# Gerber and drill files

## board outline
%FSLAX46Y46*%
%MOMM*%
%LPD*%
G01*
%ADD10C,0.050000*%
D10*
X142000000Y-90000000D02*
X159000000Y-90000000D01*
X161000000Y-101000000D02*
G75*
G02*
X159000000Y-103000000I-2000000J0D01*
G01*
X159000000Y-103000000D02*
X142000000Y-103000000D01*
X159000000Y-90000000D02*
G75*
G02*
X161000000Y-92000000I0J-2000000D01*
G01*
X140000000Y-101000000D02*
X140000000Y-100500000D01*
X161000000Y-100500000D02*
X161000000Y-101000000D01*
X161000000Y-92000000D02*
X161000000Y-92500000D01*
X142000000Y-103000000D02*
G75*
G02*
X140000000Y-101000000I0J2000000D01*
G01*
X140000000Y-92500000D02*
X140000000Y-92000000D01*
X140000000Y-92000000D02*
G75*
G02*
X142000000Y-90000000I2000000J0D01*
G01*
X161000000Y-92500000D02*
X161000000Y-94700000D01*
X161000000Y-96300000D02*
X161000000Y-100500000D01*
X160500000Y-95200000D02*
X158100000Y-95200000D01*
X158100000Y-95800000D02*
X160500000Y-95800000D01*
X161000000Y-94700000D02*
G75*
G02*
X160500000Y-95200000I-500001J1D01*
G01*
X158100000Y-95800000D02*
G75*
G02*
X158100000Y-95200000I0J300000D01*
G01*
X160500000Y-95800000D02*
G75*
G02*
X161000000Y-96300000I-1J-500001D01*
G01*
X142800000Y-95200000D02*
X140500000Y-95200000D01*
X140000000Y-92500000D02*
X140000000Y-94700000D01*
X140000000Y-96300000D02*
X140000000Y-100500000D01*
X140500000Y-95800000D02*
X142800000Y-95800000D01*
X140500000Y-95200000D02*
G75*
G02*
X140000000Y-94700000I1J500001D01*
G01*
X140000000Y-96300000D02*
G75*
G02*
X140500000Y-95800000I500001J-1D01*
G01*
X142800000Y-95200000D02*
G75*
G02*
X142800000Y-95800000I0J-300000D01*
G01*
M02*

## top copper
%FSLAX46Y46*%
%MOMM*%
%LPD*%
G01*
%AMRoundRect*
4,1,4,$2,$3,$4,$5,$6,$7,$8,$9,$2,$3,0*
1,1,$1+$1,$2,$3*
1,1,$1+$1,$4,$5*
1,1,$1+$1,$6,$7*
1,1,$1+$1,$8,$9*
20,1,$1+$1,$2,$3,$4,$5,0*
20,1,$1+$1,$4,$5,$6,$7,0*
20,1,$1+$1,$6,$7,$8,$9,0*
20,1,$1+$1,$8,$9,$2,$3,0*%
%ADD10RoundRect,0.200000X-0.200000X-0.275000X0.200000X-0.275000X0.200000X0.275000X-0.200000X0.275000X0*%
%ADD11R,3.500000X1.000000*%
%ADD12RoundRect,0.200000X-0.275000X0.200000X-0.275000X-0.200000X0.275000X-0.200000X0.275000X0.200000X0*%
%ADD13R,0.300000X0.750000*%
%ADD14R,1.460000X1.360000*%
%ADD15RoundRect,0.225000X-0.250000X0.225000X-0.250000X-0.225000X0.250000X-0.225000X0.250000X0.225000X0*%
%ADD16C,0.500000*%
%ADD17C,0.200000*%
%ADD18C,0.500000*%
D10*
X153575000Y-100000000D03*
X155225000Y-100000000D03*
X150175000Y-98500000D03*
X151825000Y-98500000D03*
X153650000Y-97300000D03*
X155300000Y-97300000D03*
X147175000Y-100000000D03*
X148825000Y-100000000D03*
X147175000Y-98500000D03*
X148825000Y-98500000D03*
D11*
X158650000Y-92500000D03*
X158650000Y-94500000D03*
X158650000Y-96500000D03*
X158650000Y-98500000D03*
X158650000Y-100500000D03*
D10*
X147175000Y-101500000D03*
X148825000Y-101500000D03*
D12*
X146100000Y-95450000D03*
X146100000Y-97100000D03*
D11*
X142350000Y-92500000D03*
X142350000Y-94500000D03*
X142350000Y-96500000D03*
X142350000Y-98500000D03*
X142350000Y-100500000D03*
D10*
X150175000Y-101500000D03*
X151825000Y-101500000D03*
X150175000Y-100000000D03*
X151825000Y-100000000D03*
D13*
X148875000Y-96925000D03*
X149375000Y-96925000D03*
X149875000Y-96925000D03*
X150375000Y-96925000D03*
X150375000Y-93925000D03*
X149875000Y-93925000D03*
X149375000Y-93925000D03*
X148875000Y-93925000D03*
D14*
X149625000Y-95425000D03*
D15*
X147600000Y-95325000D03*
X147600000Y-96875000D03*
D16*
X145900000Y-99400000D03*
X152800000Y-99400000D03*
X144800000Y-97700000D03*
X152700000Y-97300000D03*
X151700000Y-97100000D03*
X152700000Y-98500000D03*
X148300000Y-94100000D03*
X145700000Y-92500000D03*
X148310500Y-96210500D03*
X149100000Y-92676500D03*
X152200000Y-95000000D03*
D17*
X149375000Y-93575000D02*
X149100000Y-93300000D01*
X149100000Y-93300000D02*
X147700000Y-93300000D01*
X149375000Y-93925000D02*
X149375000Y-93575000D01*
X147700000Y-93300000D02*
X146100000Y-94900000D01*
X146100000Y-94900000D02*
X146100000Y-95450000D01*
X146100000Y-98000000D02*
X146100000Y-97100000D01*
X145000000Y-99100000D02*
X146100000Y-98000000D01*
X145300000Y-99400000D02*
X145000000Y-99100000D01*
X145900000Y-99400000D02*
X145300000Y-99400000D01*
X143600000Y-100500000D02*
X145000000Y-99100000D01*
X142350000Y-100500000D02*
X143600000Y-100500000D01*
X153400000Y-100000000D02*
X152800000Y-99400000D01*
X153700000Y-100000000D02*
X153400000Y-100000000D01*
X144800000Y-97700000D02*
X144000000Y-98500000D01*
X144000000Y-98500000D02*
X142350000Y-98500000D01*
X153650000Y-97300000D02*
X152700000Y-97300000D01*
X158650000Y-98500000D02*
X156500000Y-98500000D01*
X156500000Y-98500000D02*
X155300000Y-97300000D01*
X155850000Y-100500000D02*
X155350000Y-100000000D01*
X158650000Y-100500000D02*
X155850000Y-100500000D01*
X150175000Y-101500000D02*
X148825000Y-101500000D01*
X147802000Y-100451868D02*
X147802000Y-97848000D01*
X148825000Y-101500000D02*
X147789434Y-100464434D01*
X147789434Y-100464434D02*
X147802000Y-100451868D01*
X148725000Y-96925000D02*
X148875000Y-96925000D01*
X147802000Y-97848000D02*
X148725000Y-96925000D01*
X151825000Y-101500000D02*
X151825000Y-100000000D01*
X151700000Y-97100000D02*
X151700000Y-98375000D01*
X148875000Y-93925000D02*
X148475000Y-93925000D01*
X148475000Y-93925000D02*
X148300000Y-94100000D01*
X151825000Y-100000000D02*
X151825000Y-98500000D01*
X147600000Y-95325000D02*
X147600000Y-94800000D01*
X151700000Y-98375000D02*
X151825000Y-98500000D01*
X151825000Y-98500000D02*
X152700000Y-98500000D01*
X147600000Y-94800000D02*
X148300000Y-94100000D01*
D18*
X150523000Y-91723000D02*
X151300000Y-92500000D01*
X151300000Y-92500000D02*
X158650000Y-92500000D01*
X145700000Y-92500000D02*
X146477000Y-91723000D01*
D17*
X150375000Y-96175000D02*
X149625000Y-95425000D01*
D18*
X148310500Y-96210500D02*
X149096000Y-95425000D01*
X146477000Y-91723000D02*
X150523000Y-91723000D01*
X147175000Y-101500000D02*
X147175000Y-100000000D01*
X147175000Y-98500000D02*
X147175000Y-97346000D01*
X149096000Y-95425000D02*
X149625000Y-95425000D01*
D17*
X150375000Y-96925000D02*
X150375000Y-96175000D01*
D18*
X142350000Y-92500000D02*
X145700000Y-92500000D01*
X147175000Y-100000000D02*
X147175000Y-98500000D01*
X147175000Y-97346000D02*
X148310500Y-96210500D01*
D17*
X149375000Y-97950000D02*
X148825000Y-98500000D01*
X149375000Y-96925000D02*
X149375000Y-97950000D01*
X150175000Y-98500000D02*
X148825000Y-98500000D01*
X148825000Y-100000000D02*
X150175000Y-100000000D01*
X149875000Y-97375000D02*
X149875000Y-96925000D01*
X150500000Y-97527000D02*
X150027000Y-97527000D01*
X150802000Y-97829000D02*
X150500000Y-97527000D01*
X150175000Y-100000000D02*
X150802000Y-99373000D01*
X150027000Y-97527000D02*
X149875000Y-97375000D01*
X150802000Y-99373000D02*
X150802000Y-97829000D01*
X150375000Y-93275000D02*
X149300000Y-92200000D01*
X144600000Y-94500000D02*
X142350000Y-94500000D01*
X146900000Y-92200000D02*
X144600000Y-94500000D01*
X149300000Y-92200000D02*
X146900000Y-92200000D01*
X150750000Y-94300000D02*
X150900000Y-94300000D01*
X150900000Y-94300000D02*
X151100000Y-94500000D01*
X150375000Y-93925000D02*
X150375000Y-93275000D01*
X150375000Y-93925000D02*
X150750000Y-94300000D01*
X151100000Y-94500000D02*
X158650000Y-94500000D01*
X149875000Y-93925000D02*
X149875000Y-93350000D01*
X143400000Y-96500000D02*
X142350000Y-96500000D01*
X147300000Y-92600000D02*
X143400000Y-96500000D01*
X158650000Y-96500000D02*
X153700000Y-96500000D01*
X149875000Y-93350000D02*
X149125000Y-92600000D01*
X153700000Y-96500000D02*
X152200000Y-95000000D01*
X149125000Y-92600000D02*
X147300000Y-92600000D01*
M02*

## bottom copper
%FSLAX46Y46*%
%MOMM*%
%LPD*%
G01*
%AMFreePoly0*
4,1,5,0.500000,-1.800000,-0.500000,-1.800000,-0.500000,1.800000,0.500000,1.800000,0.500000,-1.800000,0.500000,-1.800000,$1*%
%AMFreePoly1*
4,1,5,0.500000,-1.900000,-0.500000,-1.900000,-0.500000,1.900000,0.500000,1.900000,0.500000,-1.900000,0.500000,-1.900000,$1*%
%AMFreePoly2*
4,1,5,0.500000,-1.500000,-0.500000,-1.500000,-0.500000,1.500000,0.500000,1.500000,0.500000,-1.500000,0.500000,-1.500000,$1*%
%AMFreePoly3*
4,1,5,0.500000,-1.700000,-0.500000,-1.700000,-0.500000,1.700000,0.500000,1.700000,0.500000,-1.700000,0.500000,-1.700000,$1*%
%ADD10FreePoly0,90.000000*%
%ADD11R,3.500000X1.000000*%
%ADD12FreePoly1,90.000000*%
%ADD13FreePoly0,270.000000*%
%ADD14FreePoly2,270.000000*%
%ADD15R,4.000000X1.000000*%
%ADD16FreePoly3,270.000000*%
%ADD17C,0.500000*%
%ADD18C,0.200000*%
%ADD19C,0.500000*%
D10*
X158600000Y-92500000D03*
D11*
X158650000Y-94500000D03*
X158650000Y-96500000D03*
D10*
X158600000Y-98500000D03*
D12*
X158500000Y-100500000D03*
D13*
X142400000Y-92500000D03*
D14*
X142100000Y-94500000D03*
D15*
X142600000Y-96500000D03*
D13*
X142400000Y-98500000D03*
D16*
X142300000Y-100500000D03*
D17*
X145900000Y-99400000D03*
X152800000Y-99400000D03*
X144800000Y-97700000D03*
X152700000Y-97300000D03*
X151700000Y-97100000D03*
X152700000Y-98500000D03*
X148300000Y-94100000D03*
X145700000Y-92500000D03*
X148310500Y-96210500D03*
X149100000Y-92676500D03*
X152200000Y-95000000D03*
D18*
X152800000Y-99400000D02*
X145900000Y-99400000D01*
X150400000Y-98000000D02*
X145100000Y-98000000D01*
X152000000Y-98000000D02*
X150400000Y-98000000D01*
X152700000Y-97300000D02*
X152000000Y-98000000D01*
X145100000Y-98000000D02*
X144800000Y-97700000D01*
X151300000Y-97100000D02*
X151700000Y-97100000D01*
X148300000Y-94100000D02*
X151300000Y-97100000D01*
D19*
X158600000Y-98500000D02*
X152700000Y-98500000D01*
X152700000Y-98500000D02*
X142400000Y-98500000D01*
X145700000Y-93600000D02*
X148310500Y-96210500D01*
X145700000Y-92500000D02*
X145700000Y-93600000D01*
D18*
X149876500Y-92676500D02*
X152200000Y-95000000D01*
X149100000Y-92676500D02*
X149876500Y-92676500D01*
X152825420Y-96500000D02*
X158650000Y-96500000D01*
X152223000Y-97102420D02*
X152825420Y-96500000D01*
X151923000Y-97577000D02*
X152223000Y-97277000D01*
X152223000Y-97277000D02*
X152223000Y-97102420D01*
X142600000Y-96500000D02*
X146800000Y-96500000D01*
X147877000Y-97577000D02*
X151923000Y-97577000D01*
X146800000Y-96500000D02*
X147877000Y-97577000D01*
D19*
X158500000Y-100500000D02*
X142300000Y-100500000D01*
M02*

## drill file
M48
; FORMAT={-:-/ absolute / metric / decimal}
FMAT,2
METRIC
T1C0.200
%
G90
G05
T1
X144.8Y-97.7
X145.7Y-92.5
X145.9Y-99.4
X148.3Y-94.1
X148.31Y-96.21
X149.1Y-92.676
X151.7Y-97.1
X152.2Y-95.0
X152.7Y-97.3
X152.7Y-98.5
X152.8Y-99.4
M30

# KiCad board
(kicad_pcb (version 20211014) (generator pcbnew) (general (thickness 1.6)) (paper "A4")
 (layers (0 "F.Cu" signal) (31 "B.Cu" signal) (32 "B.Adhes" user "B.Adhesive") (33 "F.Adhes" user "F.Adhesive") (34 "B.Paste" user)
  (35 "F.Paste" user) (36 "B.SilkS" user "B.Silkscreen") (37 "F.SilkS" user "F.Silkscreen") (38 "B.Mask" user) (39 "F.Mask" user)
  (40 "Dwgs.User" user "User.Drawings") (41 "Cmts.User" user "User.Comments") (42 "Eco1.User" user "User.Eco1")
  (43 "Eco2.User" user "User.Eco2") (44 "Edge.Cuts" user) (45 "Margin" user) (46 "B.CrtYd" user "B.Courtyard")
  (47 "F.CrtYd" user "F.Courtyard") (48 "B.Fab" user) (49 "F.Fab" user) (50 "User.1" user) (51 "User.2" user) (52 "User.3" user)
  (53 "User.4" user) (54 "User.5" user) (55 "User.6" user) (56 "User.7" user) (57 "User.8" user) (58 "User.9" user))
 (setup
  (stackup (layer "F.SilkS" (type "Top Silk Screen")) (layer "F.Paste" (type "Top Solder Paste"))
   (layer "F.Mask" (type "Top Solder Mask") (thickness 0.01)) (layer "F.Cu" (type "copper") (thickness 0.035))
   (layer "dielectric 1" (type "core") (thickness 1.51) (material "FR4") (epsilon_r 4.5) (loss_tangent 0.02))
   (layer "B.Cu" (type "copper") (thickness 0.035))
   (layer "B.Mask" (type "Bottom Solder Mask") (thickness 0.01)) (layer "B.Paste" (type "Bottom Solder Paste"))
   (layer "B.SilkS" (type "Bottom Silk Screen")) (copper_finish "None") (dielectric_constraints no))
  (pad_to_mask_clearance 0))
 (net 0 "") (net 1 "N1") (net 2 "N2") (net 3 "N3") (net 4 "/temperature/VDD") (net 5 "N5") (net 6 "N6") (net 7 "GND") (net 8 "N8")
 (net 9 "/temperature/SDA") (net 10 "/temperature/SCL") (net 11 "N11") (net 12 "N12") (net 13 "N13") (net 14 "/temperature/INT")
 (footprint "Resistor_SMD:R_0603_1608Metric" (layer "F.Cu") (at 154.4 100)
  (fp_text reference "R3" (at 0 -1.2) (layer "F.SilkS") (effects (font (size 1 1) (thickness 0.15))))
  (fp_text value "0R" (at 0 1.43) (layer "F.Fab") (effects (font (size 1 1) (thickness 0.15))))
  (pad "1" smd roundrect (at -0.825 0) (size 0.8 0.95) (layers "F.Cu" "F.Paste" "F.Mask") (roundrect_rratio 0.25) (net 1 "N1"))
  (pad "2" smd roundrect (at 0.825 0) (size 0.8 0.95) (layers "F.Cu" "F.Paste" "F.Mask") (roundrect_rratio 0.25) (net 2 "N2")))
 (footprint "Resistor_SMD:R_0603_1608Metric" (layer "F.Cu") (at 151 98.5)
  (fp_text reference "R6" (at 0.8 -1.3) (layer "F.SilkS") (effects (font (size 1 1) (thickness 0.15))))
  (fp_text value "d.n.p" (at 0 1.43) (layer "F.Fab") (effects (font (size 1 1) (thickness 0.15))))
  (pad "1" smd roundrect (at -0.825 0) (size 0.8 0.95) (layers "F.Cu" "F.Paste" "F.Mask") (roundrect_rratio 0.25) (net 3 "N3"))
  (pad "2" smd roundrect (at 0.825 0) (size 0.8 0.95) (layers "F.Cu" "F.Paste" "F.Mask") (roundrect_rratio 0.25) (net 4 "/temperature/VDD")))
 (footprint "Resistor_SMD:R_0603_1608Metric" (layer "F.Cu") (at 154.475 97.3)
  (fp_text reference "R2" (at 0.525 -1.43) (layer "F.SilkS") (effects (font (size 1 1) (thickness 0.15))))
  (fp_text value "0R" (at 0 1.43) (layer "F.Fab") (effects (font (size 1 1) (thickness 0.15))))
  (pad "1" smd roundrect (at -0.825 0) (size 0.8 0.95) (layers "F.Cu" "F.Paste" "F.Mask") (roundrect_rratio 0.25) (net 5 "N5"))
  (pad "2" smd roundrect (at 0.825 0) (size 0.8 0.95) (layers "F.Cu" "F.Paste" "F.Mask") (roundrect_rratio 0.25) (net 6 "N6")))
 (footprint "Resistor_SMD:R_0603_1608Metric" (layer "F.Cu") (at 148 100)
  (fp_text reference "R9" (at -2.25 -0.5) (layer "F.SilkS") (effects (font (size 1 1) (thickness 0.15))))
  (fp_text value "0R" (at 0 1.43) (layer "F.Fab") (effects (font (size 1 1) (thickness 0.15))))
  (pad "1" smd roundrect (at -0.825 0) (size 0.8 0.95) (layers "F.Cu" "F.Paste" "F.Mask") (roundrect_rratio 0.25) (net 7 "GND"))
  (pad "2" smd roundrect (at 0.825 0) (size 0.8 0.95) (layers "F.Cu" "F.Paste" "F.Mask") (roundrect_rratio 0.25) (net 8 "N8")))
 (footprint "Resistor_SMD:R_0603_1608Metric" (layer "F.Cu") (at 148 98.5)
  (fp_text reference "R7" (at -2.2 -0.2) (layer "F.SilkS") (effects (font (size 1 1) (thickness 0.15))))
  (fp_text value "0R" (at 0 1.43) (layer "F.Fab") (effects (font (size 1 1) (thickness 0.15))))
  (pad "1" smd roundrect (at -0.825 0) (size 0.8 0.95) (layers "F.Cu" "F.Paste" "F.Mask") (roundrect_rratio 0.25) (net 7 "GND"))
  (pad "2" smd roundrect (at 0.825 0) (size 0.8 0.95) (layers "F.Cu" "F.Paste" "F.Mask") (roundrect_rratio 0.25) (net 3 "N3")))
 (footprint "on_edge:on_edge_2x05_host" (layer "F.Cu") (at 161 96.5 -90)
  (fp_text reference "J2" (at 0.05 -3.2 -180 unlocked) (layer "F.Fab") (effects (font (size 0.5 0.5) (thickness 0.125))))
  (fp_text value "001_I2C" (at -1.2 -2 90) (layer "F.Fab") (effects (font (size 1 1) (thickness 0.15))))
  (fp_line (start -4 0) (end -1.8 0) (layer "Edge.Cuts") (width 0.05))
  (fp_line (start -0.2 0) (end 4 0) (layer "Edge.Cuts") (width 0.05))
  (fp_line (start -1.3 0.5) (end -1.3 2.9) (layer "Edge.Cuts") (width 0.05))
  (fp_line (start -0.7 2.9) (end -0.7 0.5) (layer "Edge.Cuts") (width 0.05))
  (fp_arc (start -1.8 0) (mid -1.446447 0.146447) (end -1.3 0.5) (layer "Edge.Cuts") (width 0.05))
  (fp_arc (start -0.7 2.9) (mid -1 3.2) (end -1.3 2.9) (layer "Edge.Cuts") (width 0.05))
  (fp_arc (start -0.7 0.5) (mid -0.553553 0.146447) (end -0.2 0) (layer "Edge.Cuts") (width 0.05))
  (pad "1" smd rect (at -4 2.35 270) (size 1 3.5) (layers "F.Cu" "F.Mask") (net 7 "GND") (zone_connect 0))
  (pad "2" smd rect (at -2 2.35 270) (size 1 3.5) (layers "F.Cu" "F.Mask") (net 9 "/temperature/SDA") (zone_connect 0))
  (pad "3" smd rect (at 0 2.35 270) (size 1 3.5) (layers "F.Cu" "F.Mask") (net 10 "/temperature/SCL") (zone_connect 0))
  (pad "4" smd rect (at 2 2.35 270) (size 1 3.5) (layers "F.Cu" "F.Mask") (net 6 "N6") (zone_connect 0))
  (pad "5" smd rect (at 4 2.35 270) (size 1 3.5) (layers "F.Cu" "F.Mask") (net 2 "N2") (zone_connect 0))
  (pad "6" smd custom (at -4 2.4 90) (size 1 3.6) (layers "B.Cu" "B.Mask") (zone_connect 0) (options (clearance outline) (anchor rect))
   (primitives))
  (pad "7" smd rect (at -2 2.35 90) (size 1 3.5) (layers "B.Cu" "B.Mask") (zone_connect 0))
  (pad "8" smd rect (at 0 2.35 90) (size 1 3.5) (layers "B.Cu" "B.Mask") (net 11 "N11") (zone_connect 0))
  (pad "9" smd custom (at 2 2.4 90) (size 1 3.6) (layers "B.Cu" "B.Mask") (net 4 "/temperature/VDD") (zone_connect 0)
   (options (clearance outline) (anchor rect)) (primitives))
  (pad "10" smd custom (at 4 2.5 90) (size 1 3.8) (layers "B.Cu" "B.Mask") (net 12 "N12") (zone_connect 0)
   (options (clearance outline) (anchor rect)) (primitives)))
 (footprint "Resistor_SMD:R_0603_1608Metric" (layer "F.Cu") (at 148 101.5)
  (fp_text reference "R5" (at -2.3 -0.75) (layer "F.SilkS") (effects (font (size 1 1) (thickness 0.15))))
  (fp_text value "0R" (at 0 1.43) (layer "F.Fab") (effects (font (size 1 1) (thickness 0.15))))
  (pad "1" smd roundrect (at -0.825 0) (size 0.8 0.95) (layers "F.Cu" "F.Paste" "F.Mask") (roundrect_rratio 0.25) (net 7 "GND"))
  (pad "2" smd roundrect (at 0.825 0) (size 0.8 0.95) (layers "F.Cu" "F.Paste" "F.Mask") (roundrect_rratio 0.25) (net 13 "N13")))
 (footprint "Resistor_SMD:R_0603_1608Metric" (layer "F.Cu") (at 146.1 96.275 -90)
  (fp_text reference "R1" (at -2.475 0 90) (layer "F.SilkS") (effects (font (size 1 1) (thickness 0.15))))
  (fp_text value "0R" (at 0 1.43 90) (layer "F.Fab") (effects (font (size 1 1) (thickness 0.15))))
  (pad "1" smd roundrect (at -0.825 0 270) (size 0.8 0.95) (layers "F.Cu" "F.Paste" "F.Mask") (roundrect_rratio 0.25)
   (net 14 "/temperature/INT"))
  (pad "2" smd roundrect (at 0.825 0 270) (size 0.8 0.95) (layers "F.Cu" "F.Paste" "F.Mask") (roundrect_rratio 0.25) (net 1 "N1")))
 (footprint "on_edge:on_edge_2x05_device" (layer "F.Cu") (at 140 96.5 -90)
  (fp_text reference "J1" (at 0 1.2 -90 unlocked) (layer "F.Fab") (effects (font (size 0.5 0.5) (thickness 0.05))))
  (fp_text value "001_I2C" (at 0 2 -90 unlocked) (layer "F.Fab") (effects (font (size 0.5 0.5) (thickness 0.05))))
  (fp_line (start -1.3 -2.8) (end -1.3 -0.5) (layer "Edge.Cuts") (width 0.05))
  (fp_line (start -4 0) (end -1.8 0) (layer "Edge.Cuts") (width 0.05))
  (fp_line (start -0.2 0) (end 4 0) (layer "Edge.Cuts") (width 0.05))
  (fp_line (start -0.7 -0.5) (end -0.7 -2.8) (layer "Edge.Cuts") (width 0.05))
  (fp_arc (start -1.3 -0.5) (mid -1.446447 -0.146447) (end -1.8 0) (layer "Edge.Cuts") (width 0.05))
  (fp_arc (start -0.2 0) (mid -0.553553 -0.146447) (end -0.7 -0.5) (layer "Edge.Cuts") (width 0.05))
  (fp_arc (start -1.3 -2.8) (mid -1 -3.1) (end -0.7 -2.8) (layer "Edge.Cuts") (width 0.05))
  (pad "1" smd rect (at -4 -2.35 90) (size 1 3.5) (layers "F.Cu" "F.Mask") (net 7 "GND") (zone_connect 0))
  (pad "2" smd rect (at -2 -2.35 270) (size 1 3.5) (layers "F.Cu" "F.Mask") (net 9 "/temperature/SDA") (zone_connect 0))
  (pad "3" smd rect (at 0 -2.35 270) (size 1 3.5) (layers "F.Cu" "F.Mask") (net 10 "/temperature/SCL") (zone_connect 0))
  (pad "4" smd rect (at 2 -2.35 90) (size 1 3.5) (layers "F.Cu" "F.Mask") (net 5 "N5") (zone_connect 0))
  (pad "5" smd rect (at 4 -2.35 90) (size 1 3.5) (layers "F.Cu" "F.Mask") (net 1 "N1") (zone_connect 0))
  (pad "6" smd custom (at -4 -2.4 270) (size 1 3.6) (layers "B.Cu" "B.Mask") (zone_connect 0) (options (clearance outline) (anchor rect))
   (primitives))
  (pad "7" smd custom (at -2 -2.1 270) (size 1 3) (layers "B.Cu" "B.Mask") (zone_connect 0) (options (clearance outline) (anchor rect))
   (primitives))
  (pad "8" smd rect (at 0 -2.6 270) (size 1 4) (layers "B.Cu" "B.Mask") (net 11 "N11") (zone_connect 0))
  (pad "9" smd custom (at 2 -2.4 270) (size 1 3.6) (layers "B.Cu" "B.Mask") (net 4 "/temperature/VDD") (zone_connect 0)
   (options (clearance outline) (anchor rect)) (primitives))
  (pad "10" smd custom (at 4 -2.3 270) (size 1 3.4) (layers "B.Cu" "B.Mask") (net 12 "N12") (zone_connect 0)
   (options (clearance outline) (anchor rect)) (primitives)))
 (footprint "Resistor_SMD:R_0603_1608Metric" (layer "F.Cu") (at 151 101.5)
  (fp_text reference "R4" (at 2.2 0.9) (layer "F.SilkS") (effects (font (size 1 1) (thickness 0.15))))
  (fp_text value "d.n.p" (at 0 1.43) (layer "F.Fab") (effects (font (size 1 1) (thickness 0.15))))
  (pad "1" smd roundrect (at -0.825 0) (size 0.8 0.95) (layers "F.Cu" "F.Paste" "F.Mask") (roundrect_rratio 0.25) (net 13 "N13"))
  (pad "2" smd roundrect (at 0.825 0) (size 0.8 0.95) (layers "F.Cu" "F.Paste" "F.Mask") (roundrect_rratio 0.25) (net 4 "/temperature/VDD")))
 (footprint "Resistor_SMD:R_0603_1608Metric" (layer "F.Cu") (at 151 100)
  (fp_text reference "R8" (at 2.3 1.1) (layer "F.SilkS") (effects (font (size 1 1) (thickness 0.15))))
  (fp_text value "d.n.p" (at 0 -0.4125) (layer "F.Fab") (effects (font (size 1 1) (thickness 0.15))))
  (pad "1" smd roundrect (at -0.825 0) (size 0.8 0.95) (layers "F.Cu" "F.Paste" "F.Mask") (roundrect_rratio 0.25) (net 8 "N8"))
  (pad "2" smd roundrect (at 0.825 0) (size 0.8 0.95) (layers "F.Cu" "F.Paste" "F.Mask") (roundrect_rratio 0.25) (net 4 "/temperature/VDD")))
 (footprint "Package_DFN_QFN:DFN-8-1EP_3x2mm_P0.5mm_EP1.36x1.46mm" (layer "F.Cu") (at 149.625 95.425 90)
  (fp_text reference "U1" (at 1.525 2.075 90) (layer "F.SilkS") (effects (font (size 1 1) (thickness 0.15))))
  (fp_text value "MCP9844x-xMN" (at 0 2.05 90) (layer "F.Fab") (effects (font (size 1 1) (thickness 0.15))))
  (pad "" smd rect (at 0.325 0.375 90) (size 0.5 0.6) (layers "F.Paste"))
  (pad "" smd rect (at -0.325 -0.375 90) (size 0.5 0.6) (layers "F.Paste"))
  (pad "" smd rect (at 0.325 -0.375 90) (size 0.5 0.6) (layers "F.Paste"))
  (pad "" smd rect (at -0.325 0.375 90) (size 0.5 0.6) (layers "F.Paste"))
  (pad "1" smd rect (at -1.5 -0.75 90) (size 0.75 0.3) (layers "F.Cu" "F.Paste" "F.Mask") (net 13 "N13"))
  (pad "2" smd rect (at -1.5 -0.25 90) (size 0.75 0.3) (layers "F.Cu" "F.Paste" "F.Mask") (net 3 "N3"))
  (pad "3" smd rect (at -1.5 0.25 90) (size 0.75 0.3) (layers "F.Cu" "F.Paste" "F.Mask") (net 8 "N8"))
  (pad "4" smd rect (at -1.5 0.75 90) (size 0.75 0.3) (layers "F.Cu" "F.Paste" "F.Mask") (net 7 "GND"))
  (pad "5" smd rect (at 1.5 0.75 90) (size 0.75 0.3) (layers "F.Cu" "F.Paste" "F.Mask") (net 9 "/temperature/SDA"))
  (pad "6" smd rect (at 1.5 0.25 90) (size 0.75 0.3) (layers "F.Cu" "F.Paste" "F.Mask") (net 10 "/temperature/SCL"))
  (pad "7" smd rect (at 1.5 -0.25 90) (size 0.75 0.3) (layers "F.Cu" "F.Paste" "F.Mask") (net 14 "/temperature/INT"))
  (pad "8" smd rect (at 1.5 -0.75 90) (size 0.75 0.3) (layers "F.Cu" "F.Paste" "F.Mask") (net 4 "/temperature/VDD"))
  (pad "9" smd rect (at 0 0 90) (size 1.36 1.46) (layers "F.Cu" "F.Mask") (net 7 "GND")))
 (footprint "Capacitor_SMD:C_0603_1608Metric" (layer "F.Cu") (at 147.6 96.1 -90)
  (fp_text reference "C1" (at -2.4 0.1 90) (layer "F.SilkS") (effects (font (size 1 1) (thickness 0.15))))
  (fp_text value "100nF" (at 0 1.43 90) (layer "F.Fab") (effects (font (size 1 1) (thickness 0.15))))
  (pad "1" smd roundrect (at -0.775 0 270) (size 0.9 0.95) (layers "F.Cu" "F.Paste" "F.Mask") (roundrect_rratio 0.25)
   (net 4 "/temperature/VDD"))
  (pad "2" smd roundrect (at 0.775 0 270) (size 0.9 0.95) (layers "F.Cu" "F.Paste" "F.Mask") (roundrect_rratio 0.25) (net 7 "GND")))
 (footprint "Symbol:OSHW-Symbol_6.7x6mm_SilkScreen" (layer "B.Cu") (at 150 99 180)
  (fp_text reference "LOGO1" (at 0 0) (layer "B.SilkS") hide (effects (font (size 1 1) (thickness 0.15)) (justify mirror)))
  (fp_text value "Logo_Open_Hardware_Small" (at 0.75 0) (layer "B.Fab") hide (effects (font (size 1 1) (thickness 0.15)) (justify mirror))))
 (gr_line (start 142 90) (end 159 90) (layer "Edge.Cuts") (width 0.05))
 (gr_arc (start 161 101) (mid 160.414214 102.414214) (end 159 103) (layer "Edge.Cuts") (width 0.05))
 (gr_line (start 159 103) (end 142 103) (layer "Edge.Cuts") (width 0.05))
 (gr_arc (start 159 90) (mid 160.414214 90.585786) (end 161 92) (layer "Edge.Cuts") (width 0.05))
 (gr_line (start 140 101) (end 140 100.5) (layer "Edge.Cuts") (width 0.05))
 (gr_line (start 161 100.5) (end 161 101) (layer "Edge.Cuts") (width 0.05))
 (gr_line (start 161 92) (end 161 92.5) (layer "Edge.Cuts") (width 0.05))
 (gr_arc (start 142 103) (mid 140.585786 102.414214) (end 140 101) (layer "Edge.Cuts") (width 0.05))
 (gr_line (start 140 92.5) (end 140 92) (layer "Edge.Cuts") (width 0.05))
 (gr_arc (start 140 92) (mid 140.585786 90.585786) (end 142 90) (layer "Edge.Cuts") (width 0.05))
 (segment (start 149.375 93.575) (end 149.1 93.3) (width 0.2) (layer "F.Cu") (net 14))
 (segment (start 149.1 93.3) (end 147.7 93.3) (width 0.2) (layer "F.Cu") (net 14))
 (segment (start 149.375 93.925) (end 149.375 93.575) (width 0.2) (layer "F.Cu") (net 14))
 (segment (start 147.7 93.3) (end 146.1 94.9) (width 0.2) (layer "F.Cu") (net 14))
 (segment (start 146.1 94.9) (end 146.1 95.45) (width 0.2) (layer "F.Cu") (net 14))
 (segment (start 146.1 98) (end 146.1 97.1) (width 0.2) (layer "F.Cu") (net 1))
 (segment (start 145 99.1) (end 146.1 98) (width 0.2) (layer "F.Cu") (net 1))
 (segment (start 145.3 99.4) (end 145 99.1) (width 0.2) (layer "F.Cu") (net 1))
 (segment (start 145.9 99.4) (end 145.3 99.4) (width 0.2) (layer "F.Cu") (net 1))
 (segment (start 143.6 100.5) (end 145 99.1) (width 0.2) (layer "F.Cu") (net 1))
 (segment (start 142.35 100.5) (end 143.6 100.5) (width 0.2) (layer "F.Cu") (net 1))
 (segment (start 153.4 100) (end 152.8 99.4) (width 0.2) (layer "F.Cu") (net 1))
 (segment (start 153.7 100) (end 153.4 100) (width 0.2) (layer "F.Cu") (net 1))
 (via (at 145.9 99.4) (size 0.5) (drill 0.2) (layers "F.Cu" "B.Cu") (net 1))
 (via (at 152.8 99.4) (size 0.5) (drill 0.2) (layers "F.Cu" "B.Cu") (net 1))
 (segment (start 152.8 99.4) (end 145.9 99.4) (width 0.2) (layer "B.Cu") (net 1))
 (segment (start 144.8 97.7) (end 144 98.5) (width 0.2) (layer "F.Cu") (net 5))
 (segment (start 144 98.5) (end 142.35 98.5) (width 0.2) (layer "F.Cu") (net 5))
 (segment (start 153.65 97.3) (end 152.7 97.3) (width 0.2) (layer "F.Cu") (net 5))
 (via (at 144.8 97.7) (size 0.5) (drill 0.2) (layers "F.Cu" "B.Cu") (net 5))
 (via (at 152.7 97.3) (size 0.5) (drill 0.2) (layers "F.Cu" "B.Cu") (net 5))
 (segment (start 150.4 98) (end 145.1 98) (width 0.2) (layer "B.Cu") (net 5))
 (segment (start 152 98) (end 150.4 98) (width 0.2) (layer "B.Cu") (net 5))
 (segment (start 152.7 97.3) (end 152 98) (width 0.2) (layer "B.Cu") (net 5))
 (segment (start 145.1 98) (end 144.8 97.7) (width 0.2) (layer "B.Cu") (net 5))
 (segment (start 158.65 98.5) (end 156.5 98.5) (width 0.2) (layer "F.Cu") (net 6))
 (segment (start 156.5 98.5) (end 155.3 97.3) (width 0.2) (layer "F.Cu") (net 6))
 (segment (start 155.85 100.5) (end 155.35 100) (width 0.2) (layer "F.Cu") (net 2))
 (segment (start 158.65 100.5) (end 155.85 100.5) (width 0.2) (layer "F.Cu") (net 2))
 (segment (start 150.175 101.5) (end 148.825 101.5) (width 0.2) (layer "F.Cu") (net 13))
 (segment (start 147.802 100.451868) (end 147.802 97.848) (width 0.2) (layer "F.Cu") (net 13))
 (segment (start 148.825 101.5) (end 147.789434 100.464434) (width 0.2) (layer "F.Cu") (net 13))
 (segment (start 147.789434 100.464434) (end 147.802 100.451868) (width 0.2) (layer "F.Cu") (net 13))
 (segment (start 148.725 96.925) (end 148.875 96.925) (width 0.2) (layer "F.Cu") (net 13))
 (segment (start 147.802 97.848) (end 148.725 96.925) (width 0.2) (layer "F.Cu") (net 13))
 (segment (start 151.825 101.5) (end 151.825 100) (width 0.2) (layer "F.Cu") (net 4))
 (segment (start 151.7 97.1) (end 151.7 98.375) (width 0.2) (layer "F.Cu") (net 4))
 (segment (start 148.875 93.925) (end 148.475 93.925) (width 0.2) (layer "F.Cu") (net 4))
 (segment (start 148.475 93.925) (end 148.3 94.1) (width 0.2) (layer "F.Cu") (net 4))
 (segment (start 151.825 100) (end 151.825 98.5) (width 0.2) (layer "F.Cu") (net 4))
 (segment (start 147.6 95.325) (end 147.6 94.8) (width 0.2) (layer "F.Cu") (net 4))
 (segment (start 151.7 98.375) (end 151.825 98.5) (width 0.2) (layer "F.Cu") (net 4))
 (segment (start 151.825 98.5) (end 152.7 98.5) (width 0.2) (layer "F.Cu") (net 4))
 (segment (start 147.6 94.8) (end 148.3 94.1) (width 0.2) (layer "F.Cu") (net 4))
 (via (at 151.7 97.1) (size 0.5) (drill 0.2) (layers "F.Cu" "B.Cu") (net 4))
 (via (at 152.7 98.5) (size 0.5) (drill 0.2) (layers "F.Cu" "B.Cu") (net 4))
 (via (at 148.3 94.1) (size 0.5) (drill 0.2) (layers "F.Cu" "B.Cu") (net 4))
 (segment (start 151.3 97.1) (end 151.7 97.1) (width 0.2) (layer "B.Cu") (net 4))
 (segment (start 148.3 94.1) (end 151.3 97.1) (width 0.2) (layer "B.Cu") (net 4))
 (segment (start 158.6 98.5) (end 152.7 98.5) (width 0.5) (layer "B.Cu") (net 4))
 (segment (start 152.7 98.5) (end 142.4 98.5) (width 0.5) (layer "B.Cu") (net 4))
 (segment (start 150.523 91.723) (end 151.3 92.5) (width 0.5) (layer "F.Cu") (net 7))
 (segment (start 151.3 92.5) (end 158.65 92.5) (width 0.5) (layer "F.Cu") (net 7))
 (segment (start 145.7 92.5) (end 146.477 91.723) (width 0.5) (layer "F.Cu") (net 7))
 (segment (start 150.375 96.175) (end 149.625 95.425) (width 0.2) (layer "F.Cu") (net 7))
 (segment (start 148.3105 96.2105) (end 149.096 95.425) (width 0.5) (layer "F.Cu") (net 7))
 (segment (start 146.477 91.723) (end 150.523 91.723) (width 0.5) (layer "F.Cu") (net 7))
 (segment (start 147.175 101.5) (end 147.175 100) (width 0.5) (layer "F.Cu") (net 7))
 (segment (start 147.175 98.5) (end 147.175 97.346) (width 0.5) (layer "F.Cu") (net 7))
 (segment (start 149.096 95.425) (end 149.625 95.425) (width 0.5) (layer "F.Cu") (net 7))
 (segment (start 150.375 96.925) (end 150.375 96.175) (width 0.2) (layer "F.Cu") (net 7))
 (segment (start 142.35 92.5) (end 145.7 92.5) (width 0.5) (layer "F.Cu") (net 7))
 (segment (start 147.175 100) (end 147.175 98.5) (width 0.5) (layer "F.Cu") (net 7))
 (segment (start 147.175 97.346) (end 148.3105 96.2105) (width 0.5) (layer "F.Cu") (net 7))
 (via (at 145.7 92.5) (size 0.5) (drill 0.2) (layers "F.Cu" "B.Cu") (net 7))
 (via (at 148.3105 96.2105) (size 0.5) (drill 0.2) (layers "F.Cu" "B.Cu") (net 7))
 (segment (start 145.7 93.6) (end 148.3105 96.2105) (width 0.5) (layer "B.Cu") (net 7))
 (segment (start 145.7 92.5) (end 145.7 93.6) (width 0.5) (layer "B.Cu") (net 7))
 (segment (start 149.375 97.95) (end 148.825 98.5) (width 0.2) (layer "F.Cu") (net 3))
 (segment (start 149.375 96.925) (end 149.375 97.95) (width 0.2) (layer "F.Cu") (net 3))
 (segment (start 150.175 98.5) (end 148.825 98.5) (width 0.2) (layer "F.Cu") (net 3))
 (segment (start 148.825 100) (end 150.175 100) (width 0.2) (layer "F.Cu") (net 8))
 (segment (start 149.875 97.375) (end 149.875 96.925) (width 0.2) (layer "F.Cu") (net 8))
 (segment (start 150.5 97.527) (end 150.027 97.527) (width 0.2) (layer "F.Cu") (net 8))
 (segment (start 150.802 97.829) (end 150.5 97.527) (width 0.2) (layer "F.Cu") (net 8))
 (segment (start 150.175 100) (end 150.802 99.373) (width 0.2) (layer "F.Cu") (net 8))
 (segment (start 150.027 97.527) (end 149.875 97.375) (width 0.2) (layer "F.Cu") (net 8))
 (segment (start 150.802 99.373) (end 150.802 97.829) (width 0.2) (layer "F.Cu") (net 8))
 (segment (start 150.375 93.275) (end 149.3 92.2) (width 0.2) (layer "F.Cu") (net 9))
 (segment (start 144.6 94.5) (end 142.35 94.5) (width 0.2) (layer "F.Cu") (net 9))
 (segment (start 146.9 92.2) (end 144.6 94.5) (width 0.2) (layer "F.Cu") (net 9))
 (segment (start 149.3 92.2) (end 146.9 92.2) (width 0.2) (layer "F.Cu") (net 9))
 (segment (start 150.75 94.3) (end 150.9 94.3) (width 0.2) (layer "F.Cu") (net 9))
 (segment (start 150.9 94.3) (end 151.1 94.5) (width 0.2) (layer "F.Cu") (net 9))
 (segment (start 150.375 93.925) (end 150.375 93.275) (width 0.2) (layer "F.Cu") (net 9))
 (segment (start 150.375 93.925) (end 150.75 94.3) (width 0.2) (layer "F.Cu") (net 9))
 (segment (start 151.1 94.5) (end 158.65 94.5) (width 0.2) (layer "F.Cu") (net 9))
 (segment (start 149.875 93.925) (end 149.875 93.35) (width 0.2) (layer "F.Cu") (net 10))
 (segment (start 143.4 96.5) (end 142.35 96.5) (width 0.2) (layer "F.Cu") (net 10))
 (segment (start 147.3 92.6) (end 143.4 96.5) (width 0.2) (layer "F.Cu") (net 10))
 (segment (start 158.65 96.5) (end 153.7 96.5) (width 0.2) (layer "F.Cu") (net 10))
 (segment (start 149.875 93.35) (end 149.125 92.6) (width 0.2) (layer "F.Cu") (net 10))
 (segment (start 153.7 96.5) (end 152.2 95) (width 0.2) (layer "F.Cu") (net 10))
 (segment (start 149.125 92.6) (end 147.3 92.6) (width 0.2) (layer "F.Cu") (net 10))
 (via (at 149.1 92.6765) (size 0.5) (drill 0.2) (layers "F.Cu" "B.Cu") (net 10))
 (via (at 152.2 95) (size 0.5) (drill 0.2) (layers "F.Cu" "B.Cu") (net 10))
 (segment (start 149.8765 92.6765) (end 152.2 95) (width 0.2) (layer "B.Cu") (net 10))
 (segment (start 149.1 92.6765) (end 149.8765 92.6765) (width 0.2) (layer "B.Cu") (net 10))
 (segment (start 152.82542 96.5) (end 158.65 96.5) (width 0.2) (layer "B.Cu") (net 11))
 (segment (start 152.223 97.10242) (end 152.82542 96.5) (width 0.2) (layer "B.Cu") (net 11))
 (segment (start 151.923 97.577) (end 152.223 97.277) (width 0.2) (layer "B.Cu") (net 11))
 (segment (start 152.223 97.277) (end 152.223 97.10242) (width 0.2) (layer "B.Cu") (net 11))
 (segment (start 142.6 96.5) (end 146.8 96.5) (width 0.2) (layer "B.Cu") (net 11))
 (segment (start 147.877 97.577) (end 151.923 97.577) (width 0.2) (layer "B.Cu") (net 11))
 (segment (start 146.8 96.5) (end 147.877 97.577) (width 0.2) (layer "B.Cu") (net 11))
 (segment (start 158.5 100.5) (end 142.3 100.5) (width 0.5) (layer "B.Cu") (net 12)))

